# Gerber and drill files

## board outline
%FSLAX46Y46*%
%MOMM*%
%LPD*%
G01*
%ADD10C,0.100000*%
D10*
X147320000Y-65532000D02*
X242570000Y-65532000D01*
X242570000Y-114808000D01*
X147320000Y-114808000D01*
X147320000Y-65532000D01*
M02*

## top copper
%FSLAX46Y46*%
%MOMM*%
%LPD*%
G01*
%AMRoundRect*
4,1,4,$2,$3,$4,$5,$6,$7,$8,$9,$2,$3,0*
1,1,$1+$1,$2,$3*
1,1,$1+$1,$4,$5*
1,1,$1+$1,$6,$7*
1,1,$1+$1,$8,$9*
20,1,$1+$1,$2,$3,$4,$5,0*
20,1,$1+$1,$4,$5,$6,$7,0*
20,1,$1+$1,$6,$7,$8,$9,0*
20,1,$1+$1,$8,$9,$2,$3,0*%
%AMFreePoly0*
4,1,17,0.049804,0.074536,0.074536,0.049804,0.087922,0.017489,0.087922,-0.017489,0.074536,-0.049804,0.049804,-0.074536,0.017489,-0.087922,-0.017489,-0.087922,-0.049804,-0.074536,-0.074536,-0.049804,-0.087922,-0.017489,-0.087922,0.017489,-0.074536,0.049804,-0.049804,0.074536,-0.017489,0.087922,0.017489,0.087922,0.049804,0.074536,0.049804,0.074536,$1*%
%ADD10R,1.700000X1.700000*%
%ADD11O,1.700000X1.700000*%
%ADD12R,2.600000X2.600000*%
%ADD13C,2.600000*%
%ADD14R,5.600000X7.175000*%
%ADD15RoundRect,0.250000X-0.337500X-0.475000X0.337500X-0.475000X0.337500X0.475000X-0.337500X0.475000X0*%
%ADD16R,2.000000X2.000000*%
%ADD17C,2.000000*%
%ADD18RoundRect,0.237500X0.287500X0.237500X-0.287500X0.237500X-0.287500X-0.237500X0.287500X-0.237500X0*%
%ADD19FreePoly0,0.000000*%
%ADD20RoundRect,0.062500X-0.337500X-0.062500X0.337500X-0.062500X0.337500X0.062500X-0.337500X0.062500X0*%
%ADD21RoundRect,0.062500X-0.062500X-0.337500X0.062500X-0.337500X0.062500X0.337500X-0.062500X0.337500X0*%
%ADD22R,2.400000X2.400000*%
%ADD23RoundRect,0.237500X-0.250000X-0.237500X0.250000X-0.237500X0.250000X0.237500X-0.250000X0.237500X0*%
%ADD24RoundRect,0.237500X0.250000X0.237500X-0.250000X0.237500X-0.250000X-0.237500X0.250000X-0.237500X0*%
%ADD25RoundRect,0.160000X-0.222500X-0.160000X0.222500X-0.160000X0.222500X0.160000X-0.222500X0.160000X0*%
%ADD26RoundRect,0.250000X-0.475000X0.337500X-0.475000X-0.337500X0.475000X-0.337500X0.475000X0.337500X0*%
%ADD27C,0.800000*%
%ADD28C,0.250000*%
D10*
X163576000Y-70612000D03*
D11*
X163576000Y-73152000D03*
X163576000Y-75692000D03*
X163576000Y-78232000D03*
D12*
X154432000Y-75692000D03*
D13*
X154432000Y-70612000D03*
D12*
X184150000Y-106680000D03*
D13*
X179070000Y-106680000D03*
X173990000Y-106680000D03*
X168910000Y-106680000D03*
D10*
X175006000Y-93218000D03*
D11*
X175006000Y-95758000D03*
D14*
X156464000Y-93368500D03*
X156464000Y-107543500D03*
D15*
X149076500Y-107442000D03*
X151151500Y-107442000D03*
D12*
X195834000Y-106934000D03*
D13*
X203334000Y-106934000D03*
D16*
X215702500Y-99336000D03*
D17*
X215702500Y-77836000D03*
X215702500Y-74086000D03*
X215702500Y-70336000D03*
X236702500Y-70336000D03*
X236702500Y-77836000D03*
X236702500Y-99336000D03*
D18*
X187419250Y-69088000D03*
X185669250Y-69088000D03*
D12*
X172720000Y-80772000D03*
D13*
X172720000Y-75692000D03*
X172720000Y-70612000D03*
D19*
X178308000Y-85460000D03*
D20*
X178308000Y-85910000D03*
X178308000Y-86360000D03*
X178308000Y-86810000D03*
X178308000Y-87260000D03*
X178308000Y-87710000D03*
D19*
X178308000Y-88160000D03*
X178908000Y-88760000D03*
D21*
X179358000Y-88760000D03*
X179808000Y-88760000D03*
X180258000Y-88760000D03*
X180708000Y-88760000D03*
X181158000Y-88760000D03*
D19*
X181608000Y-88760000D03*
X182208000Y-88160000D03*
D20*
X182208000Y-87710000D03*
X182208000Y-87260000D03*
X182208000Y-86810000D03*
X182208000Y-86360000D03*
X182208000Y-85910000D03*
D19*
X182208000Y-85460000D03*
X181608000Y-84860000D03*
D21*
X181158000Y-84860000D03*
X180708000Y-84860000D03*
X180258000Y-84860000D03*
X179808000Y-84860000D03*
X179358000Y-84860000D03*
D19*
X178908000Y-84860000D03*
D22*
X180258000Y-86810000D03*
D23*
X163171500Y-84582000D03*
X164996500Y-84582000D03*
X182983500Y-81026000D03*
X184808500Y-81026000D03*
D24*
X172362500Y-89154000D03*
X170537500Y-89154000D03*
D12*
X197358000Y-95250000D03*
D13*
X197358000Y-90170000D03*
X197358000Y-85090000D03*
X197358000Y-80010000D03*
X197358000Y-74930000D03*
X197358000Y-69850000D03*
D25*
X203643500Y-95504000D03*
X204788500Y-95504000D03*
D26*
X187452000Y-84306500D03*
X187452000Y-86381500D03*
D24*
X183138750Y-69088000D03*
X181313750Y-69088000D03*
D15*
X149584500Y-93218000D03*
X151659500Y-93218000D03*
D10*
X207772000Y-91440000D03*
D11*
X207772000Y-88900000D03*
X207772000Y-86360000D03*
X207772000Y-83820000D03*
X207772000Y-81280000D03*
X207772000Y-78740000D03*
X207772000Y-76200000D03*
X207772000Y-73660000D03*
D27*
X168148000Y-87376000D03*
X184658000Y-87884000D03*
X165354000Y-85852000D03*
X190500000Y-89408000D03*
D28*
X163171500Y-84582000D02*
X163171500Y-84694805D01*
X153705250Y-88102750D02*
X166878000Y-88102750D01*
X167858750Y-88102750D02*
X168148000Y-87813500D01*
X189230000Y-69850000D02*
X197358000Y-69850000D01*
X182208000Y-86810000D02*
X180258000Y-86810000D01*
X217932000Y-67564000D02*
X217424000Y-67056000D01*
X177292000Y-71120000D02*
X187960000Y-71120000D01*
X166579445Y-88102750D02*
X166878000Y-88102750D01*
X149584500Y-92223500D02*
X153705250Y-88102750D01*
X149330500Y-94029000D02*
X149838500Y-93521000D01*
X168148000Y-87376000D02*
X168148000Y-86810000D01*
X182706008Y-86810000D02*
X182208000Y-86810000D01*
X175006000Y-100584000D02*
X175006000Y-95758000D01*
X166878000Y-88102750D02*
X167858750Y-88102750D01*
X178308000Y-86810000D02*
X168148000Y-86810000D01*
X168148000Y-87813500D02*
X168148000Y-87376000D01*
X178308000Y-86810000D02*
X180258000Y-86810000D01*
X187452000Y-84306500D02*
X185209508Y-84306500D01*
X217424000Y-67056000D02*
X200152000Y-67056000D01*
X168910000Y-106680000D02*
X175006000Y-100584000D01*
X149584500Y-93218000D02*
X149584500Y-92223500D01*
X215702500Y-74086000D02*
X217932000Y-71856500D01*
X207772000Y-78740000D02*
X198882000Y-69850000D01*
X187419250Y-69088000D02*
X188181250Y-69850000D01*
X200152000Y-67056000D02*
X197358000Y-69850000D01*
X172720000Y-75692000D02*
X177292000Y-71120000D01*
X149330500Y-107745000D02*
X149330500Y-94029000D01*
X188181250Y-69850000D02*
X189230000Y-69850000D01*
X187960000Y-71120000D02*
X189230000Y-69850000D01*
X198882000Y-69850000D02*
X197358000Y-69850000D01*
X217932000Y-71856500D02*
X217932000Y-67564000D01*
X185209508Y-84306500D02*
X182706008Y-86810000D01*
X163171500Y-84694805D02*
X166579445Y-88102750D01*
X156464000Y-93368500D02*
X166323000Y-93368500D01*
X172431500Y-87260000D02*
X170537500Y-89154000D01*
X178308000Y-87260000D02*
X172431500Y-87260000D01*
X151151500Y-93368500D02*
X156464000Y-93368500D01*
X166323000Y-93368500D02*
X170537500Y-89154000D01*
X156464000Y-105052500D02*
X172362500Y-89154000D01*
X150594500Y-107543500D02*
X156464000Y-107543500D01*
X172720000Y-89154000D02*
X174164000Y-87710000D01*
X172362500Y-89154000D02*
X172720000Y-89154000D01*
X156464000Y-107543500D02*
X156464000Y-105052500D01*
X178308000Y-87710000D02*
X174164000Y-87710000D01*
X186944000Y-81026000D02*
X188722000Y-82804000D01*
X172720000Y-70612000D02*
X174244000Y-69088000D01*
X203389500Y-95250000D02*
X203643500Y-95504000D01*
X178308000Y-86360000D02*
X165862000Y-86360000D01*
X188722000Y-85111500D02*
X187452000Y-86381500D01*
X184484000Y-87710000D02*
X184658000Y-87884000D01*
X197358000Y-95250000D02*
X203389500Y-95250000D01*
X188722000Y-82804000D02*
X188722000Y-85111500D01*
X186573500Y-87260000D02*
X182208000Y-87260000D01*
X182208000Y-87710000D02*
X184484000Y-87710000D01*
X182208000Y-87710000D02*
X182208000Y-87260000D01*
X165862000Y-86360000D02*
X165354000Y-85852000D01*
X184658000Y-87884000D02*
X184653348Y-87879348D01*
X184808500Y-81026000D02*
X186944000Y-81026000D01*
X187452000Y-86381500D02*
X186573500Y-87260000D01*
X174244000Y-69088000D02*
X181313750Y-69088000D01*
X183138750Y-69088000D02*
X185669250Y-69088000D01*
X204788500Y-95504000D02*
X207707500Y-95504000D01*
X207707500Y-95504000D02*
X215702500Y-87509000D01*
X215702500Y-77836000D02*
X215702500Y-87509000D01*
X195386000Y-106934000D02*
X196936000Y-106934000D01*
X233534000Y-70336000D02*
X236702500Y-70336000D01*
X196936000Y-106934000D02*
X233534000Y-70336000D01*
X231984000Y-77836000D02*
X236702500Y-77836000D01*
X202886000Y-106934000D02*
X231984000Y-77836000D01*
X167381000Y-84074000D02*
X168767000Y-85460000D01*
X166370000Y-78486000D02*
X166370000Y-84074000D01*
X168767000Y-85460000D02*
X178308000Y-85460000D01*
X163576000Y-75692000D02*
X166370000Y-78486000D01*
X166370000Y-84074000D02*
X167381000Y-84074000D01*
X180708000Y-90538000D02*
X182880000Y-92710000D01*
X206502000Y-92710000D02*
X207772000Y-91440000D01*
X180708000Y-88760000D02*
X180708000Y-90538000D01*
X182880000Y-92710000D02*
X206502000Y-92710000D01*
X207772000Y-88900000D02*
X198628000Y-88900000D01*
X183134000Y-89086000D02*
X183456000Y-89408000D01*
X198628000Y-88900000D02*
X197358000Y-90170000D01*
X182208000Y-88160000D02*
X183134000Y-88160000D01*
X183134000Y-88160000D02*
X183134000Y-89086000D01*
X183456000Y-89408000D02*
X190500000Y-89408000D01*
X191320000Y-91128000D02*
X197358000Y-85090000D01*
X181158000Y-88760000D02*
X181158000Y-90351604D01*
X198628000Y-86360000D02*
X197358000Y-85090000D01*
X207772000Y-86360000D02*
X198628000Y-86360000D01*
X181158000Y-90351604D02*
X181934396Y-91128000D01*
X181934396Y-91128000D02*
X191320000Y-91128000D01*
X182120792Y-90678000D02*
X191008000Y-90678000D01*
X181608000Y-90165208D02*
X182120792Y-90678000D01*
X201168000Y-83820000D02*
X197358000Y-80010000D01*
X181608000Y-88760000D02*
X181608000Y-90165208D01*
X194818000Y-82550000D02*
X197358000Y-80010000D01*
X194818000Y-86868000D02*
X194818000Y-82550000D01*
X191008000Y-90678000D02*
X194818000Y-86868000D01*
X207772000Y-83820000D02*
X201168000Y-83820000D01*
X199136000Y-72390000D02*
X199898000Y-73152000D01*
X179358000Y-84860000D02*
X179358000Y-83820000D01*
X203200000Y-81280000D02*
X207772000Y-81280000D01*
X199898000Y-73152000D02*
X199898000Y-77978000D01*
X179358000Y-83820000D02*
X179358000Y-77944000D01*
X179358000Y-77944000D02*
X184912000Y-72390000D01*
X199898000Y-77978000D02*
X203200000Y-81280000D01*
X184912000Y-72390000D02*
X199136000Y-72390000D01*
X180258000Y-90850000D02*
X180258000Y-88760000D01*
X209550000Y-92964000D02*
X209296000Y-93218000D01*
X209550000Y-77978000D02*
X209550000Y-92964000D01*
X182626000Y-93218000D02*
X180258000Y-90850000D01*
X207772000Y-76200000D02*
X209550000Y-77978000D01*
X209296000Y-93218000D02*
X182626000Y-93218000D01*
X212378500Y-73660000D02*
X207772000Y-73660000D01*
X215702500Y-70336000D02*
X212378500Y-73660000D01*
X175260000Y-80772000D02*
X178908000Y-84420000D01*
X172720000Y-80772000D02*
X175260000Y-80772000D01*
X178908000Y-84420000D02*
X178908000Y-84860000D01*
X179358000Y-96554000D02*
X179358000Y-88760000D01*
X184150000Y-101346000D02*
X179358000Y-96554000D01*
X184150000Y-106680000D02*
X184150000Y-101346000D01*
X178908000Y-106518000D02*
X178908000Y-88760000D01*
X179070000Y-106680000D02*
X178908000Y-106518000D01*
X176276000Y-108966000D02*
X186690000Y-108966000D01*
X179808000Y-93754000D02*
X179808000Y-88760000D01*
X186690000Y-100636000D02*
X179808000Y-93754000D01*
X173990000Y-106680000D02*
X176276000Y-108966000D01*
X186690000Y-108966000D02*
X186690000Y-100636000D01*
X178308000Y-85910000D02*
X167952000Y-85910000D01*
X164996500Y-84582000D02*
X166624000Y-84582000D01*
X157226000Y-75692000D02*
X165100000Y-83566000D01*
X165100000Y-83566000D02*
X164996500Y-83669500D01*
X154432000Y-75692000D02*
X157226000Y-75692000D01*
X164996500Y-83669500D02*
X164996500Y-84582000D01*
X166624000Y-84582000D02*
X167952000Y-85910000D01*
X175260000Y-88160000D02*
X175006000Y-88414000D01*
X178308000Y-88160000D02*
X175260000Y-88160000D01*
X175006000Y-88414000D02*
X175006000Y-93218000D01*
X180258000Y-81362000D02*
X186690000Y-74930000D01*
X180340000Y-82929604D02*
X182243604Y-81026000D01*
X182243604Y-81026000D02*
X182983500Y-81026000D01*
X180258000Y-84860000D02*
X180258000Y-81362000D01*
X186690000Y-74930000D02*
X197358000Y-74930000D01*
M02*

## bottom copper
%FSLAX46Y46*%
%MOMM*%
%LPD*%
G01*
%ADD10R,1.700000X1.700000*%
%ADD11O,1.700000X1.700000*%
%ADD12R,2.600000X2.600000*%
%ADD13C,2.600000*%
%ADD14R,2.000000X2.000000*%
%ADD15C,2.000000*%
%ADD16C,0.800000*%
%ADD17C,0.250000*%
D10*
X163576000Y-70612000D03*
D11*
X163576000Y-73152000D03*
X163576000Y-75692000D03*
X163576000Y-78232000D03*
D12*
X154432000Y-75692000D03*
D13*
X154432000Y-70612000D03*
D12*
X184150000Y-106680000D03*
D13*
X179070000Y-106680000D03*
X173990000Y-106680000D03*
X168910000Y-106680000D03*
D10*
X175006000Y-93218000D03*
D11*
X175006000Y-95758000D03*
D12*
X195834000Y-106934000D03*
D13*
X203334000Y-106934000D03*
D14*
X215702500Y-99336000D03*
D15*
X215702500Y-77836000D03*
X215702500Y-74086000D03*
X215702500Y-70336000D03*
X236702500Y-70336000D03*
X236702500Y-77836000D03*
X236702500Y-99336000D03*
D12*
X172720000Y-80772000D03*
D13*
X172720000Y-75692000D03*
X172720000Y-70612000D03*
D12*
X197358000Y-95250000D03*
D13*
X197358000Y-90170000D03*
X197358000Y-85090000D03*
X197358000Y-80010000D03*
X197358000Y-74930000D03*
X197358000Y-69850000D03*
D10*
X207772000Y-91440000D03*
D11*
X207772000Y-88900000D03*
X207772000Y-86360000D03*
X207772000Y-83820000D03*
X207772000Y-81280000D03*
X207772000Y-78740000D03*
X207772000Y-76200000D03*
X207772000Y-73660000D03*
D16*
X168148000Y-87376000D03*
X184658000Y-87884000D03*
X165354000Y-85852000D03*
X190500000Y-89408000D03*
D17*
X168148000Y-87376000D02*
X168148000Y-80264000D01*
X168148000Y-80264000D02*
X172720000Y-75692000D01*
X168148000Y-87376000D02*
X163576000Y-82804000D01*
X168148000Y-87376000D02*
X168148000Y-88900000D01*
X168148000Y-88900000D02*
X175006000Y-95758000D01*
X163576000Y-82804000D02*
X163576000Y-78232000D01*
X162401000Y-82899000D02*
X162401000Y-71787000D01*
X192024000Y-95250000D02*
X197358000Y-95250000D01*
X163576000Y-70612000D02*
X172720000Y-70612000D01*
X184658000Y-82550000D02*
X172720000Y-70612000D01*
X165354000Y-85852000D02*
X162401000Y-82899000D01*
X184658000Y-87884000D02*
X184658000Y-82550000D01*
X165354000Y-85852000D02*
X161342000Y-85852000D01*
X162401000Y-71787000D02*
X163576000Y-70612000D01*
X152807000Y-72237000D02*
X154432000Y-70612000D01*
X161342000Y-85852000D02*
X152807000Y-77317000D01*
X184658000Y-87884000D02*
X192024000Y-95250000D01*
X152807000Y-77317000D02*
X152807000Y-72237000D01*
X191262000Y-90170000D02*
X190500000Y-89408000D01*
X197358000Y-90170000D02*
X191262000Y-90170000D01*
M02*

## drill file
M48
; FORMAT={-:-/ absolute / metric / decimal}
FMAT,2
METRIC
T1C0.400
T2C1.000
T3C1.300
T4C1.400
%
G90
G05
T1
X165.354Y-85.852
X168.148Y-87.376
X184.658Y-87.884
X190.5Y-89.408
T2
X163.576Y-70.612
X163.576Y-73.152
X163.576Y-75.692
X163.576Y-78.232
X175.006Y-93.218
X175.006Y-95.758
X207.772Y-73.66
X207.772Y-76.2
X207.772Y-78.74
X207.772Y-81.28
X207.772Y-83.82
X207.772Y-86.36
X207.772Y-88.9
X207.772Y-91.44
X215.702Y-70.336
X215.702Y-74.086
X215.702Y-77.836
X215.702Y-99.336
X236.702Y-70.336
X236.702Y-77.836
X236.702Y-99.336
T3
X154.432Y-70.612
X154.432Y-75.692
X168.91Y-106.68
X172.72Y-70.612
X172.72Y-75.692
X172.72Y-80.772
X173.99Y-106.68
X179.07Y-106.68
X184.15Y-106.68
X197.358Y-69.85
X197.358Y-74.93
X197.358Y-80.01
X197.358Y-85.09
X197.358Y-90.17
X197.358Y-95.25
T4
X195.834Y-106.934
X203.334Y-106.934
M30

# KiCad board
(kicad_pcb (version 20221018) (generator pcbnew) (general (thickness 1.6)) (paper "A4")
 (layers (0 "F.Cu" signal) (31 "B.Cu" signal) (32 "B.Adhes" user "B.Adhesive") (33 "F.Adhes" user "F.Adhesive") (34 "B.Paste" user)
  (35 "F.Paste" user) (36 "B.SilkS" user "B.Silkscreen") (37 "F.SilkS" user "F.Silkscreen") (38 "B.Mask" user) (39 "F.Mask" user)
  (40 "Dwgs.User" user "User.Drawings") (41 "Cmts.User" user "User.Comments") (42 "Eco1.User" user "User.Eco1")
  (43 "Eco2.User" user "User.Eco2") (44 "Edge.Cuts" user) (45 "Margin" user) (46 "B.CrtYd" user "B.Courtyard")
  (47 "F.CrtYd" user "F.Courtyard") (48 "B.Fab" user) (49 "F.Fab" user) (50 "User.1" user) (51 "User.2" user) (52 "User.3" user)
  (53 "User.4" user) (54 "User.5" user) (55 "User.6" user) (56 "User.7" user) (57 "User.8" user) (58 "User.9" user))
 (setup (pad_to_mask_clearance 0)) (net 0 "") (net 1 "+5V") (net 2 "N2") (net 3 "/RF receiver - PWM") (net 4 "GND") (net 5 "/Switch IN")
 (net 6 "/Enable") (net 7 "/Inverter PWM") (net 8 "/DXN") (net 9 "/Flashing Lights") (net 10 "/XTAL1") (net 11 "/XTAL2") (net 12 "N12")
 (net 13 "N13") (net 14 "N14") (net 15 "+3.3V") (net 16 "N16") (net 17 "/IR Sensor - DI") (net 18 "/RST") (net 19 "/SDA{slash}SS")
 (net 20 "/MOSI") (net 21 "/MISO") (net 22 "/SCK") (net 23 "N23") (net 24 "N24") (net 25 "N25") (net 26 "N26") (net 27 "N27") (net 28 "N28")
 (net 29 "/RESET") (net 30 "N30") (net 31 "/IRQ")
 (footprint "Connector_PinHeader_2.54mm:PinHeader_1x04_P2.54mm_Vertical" (layer "F.Cu") (at 163.576 70.612)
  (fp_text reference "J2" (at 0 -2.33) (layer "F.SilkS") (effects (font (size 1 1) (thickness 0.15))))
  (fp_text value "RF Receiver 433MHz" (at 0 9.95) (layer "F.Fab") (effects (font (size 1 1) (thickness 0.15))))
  (pad "1" thru_hole rect (at 0 0) (size 1.7 1.7) (drill 1) (layers "*.Cu" "*.Mask") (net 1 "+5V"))
  (pad "2" thru_hole oval (at 0 2.54) (size 1.7 1.7) (drill 1) (layers "*.Cu" "*.Mask") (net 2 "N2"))
  (pad "3" thru_hole oval (at 0 5.08) (size 1.7 1.7) (drill 1) (layers "*.Cu" "*.Mask") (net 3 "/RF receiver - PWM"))
  (pad "4" thru_hole oval (at 0 7.62) (size 1.7 1.7) (drill 1) (layers "*.Cu" "*.Mask") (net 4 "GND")))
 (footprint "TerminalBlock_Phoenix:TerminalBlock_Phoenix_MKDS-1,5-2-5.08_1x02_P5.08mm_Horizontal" (layer "F.Cu") (at 154.432 75.692 90)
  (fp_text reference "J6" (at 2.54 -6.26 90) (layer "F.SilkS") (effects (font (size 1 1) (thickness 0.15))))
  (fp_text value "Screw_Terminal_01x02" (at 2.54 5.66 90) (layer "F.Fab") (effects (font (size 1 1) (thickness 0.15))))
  (pad "1" thru_hole rect (at 0 0 90) (size 2.6 2.6) (drill 1.3) (layers "*.Cu" "*.Mask") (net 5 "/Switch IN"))
  (pad "2" thru_hole circle (at 5.08 0 90) (size 2.6 2.6) (drill 1.3) (layers "*.Cu" "*.Mask") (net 1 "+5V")))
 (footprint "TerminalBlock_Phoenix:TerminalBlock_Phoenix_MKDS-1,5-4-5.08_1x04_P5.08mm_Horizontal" (layer "F.Cu") (at 184.15 106.68 180)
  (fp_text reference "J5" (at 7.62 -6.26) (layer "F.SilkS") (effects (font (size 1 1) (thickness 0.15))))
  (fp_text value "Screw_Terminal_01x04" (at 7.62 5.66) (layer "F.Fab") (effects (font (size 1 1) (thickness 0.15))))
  (pad "1" thru_hole rect (at 0 0 180) (size 2.6 2.6) (drill 1.3) (layers "*.Cu" "*.Mask") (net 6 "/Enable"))
  (pad "2" thru_hole circle (at 5.08 0 180) (size 2.6 2.6) (drill 1.3) (layers "*.Cu" "*.Mask") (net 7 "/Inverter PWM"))
  (pad "3" thru_hole circle (at 10.16 0 180) (size 2.6 2.6) (drill 1.3) (layers "*.Cu" "*.Mask") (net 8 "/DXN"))
  (pad "4" thru_hole circle (at 15.24 0 180) (size 2.6 2.6) (drill 1.3) (layers "*.Cu" "*.Mask") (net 4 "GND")))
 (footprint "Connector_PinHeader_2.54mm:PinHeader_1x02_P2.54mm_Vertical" (layer "F.Cu") (at 175.006 93.218)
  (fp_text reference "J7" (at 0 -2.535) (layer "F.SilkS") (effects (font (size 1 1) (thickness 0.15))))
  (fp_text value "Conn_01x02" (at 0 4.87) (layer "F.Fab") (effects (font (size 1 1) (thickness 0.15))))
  (pad "1" thru_hole rect (at 0 0) (size 1.7 1.7) (drill 1) (layers "*.Cu" "*.Mask") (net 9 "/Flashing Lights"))
  (pad "2" thru_hole oval (at 0 2.54) (size 1.7 1.7) (drill 1) (layers "*.Cu" "*.Mask") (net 4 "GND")))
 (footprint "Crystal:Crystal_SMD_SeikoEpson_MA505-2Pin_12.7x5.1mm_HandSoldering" (layer "F.Cu") (at 156.464 100.456 -90)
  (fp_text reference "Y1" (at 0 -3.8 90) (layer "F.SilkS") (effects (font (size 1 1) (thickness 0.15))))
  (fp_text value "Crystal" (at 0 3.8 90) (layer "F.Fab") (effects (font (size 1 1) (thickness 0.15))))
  (pad "1" smd rect (at -7.0875 0 270) (size 7.175 5.6) (layers "F.Cu" "F.Paste" "F.Mask") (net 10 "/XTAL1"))
  (pad "2" smd rect (at 7.0875 0 270) (size 7.175 5.6) (layers "F.Cu" "F.Paste" "F.Mask") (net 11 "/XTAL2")))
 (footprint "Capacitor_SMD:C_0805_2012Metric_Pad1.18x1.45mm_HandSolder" (layer "F.Cu") (at 150.114 107.442)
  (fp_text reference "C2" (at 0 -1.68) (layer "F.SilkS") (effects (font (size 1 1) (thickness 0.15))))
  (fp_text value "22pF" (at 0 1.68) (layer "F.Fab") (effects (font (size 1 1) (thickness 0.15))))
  (pad "1" smd roundrect (at -1.0375 0) (size 1.175 1.45) (layers "F.Cu" "F.Paste" "F.Mask") (roundrect_rratio 0.212766) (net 4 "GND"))
  (pad "2" smd roundrect (at 1.0375 0) (size 1.175 1.45) (layers "F.Cu" "F.Paste" "F.Mask") (roundrect_rratio 0.212766) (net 11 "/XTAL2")))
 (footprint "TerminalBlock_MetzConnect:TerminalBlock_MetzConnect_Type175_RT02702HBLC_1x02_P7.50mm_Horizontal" (layer "F.Cu")
  (at 195.834 106.934)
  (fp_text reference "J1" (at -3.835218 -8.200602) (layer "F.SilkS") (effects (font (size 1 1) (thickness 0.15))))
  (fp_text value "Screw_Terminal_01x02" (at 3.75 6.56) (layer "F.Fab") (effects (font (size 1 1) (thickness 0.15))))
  (pad "1" thru_hole rect (at 0 0) (size 2.6 2.6) (drill 1.4) (layers "*.Cu" "*.Mask") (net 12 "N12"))
  (pad "2" thru_hole circle (at 7.5 0) (size 2.6 2.6) (drill 1.4) (layers "*.Cu" "*.Mask") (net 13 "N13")))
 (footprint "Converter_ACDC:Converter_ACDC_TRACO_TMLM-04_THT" (layer "F.Cu") (at 215.7025 99.336 90)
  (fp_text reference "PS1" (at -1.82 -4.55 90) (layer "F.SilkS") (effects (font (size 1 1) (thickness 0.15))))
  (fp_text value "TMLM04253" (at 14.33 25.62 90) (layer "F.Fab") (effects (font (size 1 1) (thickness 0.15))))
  (pad "1" thru_hole rect (at 0 0 90) (size 2 2) (drill 1) (layers "*.Cu" "*.Mask"))
  (pad "2" thru_hole circle (at 21.5 0 90) (size 2 2) (drill 1) (layers "*.Cu" "*.Mask") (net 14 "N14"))
  (pad "3" thru_hole circle (at 25.25 0 90) (size 2 2) (drill 1) (layers "*.Cu" "*.Mask") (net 4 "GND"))
  (pad "4" thru_hole circle (at 29 0 90) (size 2 2) (drill 1) (layers "*.Cu" "*.Mask") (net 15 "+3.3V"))
  (pad "5" thru_hole circle (at 29 21 90) (size 2 2) (drill 1) (layers "*.Cu" "*.Mask") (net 12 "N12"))
  (pad "6" thru_hole circle (at 21.5 21 90) (size 2 2) (drill 1) (layers "*.Cu" "*.Mask") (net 13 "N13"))
  (pad "7" thru_hole circle (at 0 21 90) (size 2 2) (drill 1) (layers "*.Cu" "*.Mask")))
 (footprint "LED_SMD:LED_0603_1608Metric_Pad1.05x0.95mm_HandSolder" (layer "F.Cu") (at 186.54425 69.088 180)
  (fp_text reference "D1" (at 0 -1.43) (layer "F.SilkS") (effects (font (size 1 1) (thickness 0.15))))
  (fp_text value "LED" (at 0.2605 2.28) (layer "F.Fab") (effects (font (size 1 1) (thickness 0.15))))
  (pad "1" smd roundrect (at -0.875 0 180) (size 1.05 0.95) (layers "F.Cu" "F.Paste" "F.Mask") (roundrect_rratio 0.25) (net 4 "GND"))
  (pad "2" smd roundrect (at 0.875 0 180) (size 1.05 0.95) (layers "F.Cu" "F.Paste" "F.Mask") (roundrect_rratio 0.25) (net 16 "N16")))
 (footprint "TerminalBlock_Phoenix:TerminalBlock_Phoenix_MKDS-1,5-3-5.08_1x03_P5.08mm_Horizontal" (layer "F.Cu") (at 172.72 80.772 90)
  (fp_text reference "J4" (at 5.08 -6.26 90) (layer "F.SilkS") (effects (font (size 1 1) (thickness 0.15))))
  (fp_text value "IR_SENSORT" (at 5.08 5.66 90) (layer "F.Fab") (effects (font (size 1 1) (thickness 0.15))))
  (pad "1" thru_hole rect (at 0 0 90) (size 2.6 2.6) (drill 1.3) (layers "*.Cu" "*.Mask") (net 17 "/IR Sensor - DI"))
  (pad "2" thru_hole circle (at 5.08 0 90) (size 2.6 2.6) (drill 1.3) (layers "*.Cu" "*.Mask") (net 4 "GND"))
  (pad "3" thru_hole circle (at 10.16 0 90) (size 2.6 2.6) (drill 1.3) (layers "*.Cu" "*.Mask") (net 1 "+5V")))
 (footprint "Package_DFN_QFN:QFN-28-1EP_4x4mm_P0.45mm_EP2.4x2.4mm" (layer "F.Cu") (at 180.258 86.81)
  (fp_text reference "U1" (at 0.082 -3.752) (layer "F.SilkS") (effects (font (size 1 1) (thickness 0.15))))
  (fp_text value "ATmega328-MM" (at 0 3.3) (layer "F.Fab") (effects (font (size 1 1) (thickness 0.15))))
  (pad "" smd roundrect (at -0.6 -0.6) (size 0.97 0.97) (layers "F.Paste") (roundrect_rratio 0.25))
  (pad "" smd roundrect (at -0.6 0.6) (size 0.97 0.97) (layers "F.Paste") (roundrect_rratio 0.25))
  (pad "" smd roundrect (at 0.6 -0.6) (size 0.97 0.97) (layers "F.Paste") (roundrect_rratio 0.25))
  (pad "" smd roundrect (at 0.6 0.6) (size 0.97 0.97) (layers "F.Paste") (roundrect_rratio 0.25))
  (pad "1" smd custom (at -1.95 -1.35) (size 0.179289 0.179289) (layers "F.Cu" "F.Paste" "F.Mask") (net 3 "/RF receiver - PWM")
   (thermal_bridge_angle 45) (options (clearance outline) (anchor circle)) (primitives))
  (pad "2" smd roundrect (at -1.95 -0.9) (size 0.8 0.25) (layers "F.Cu" "F.Paste" "F.Mask") (roundrect_rratio 0.25) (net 5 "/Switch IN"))
  (pad "3" smd roundrect (at -1.95 -0.45) (size 0.8 0.25) (layers "F.Cu" "F.Paste" "F.Mask") (roundrect_rratio 0.25) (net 1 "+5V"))
  (pad "4" smd roundrect (at -1.95 0) (size 0.8 0.25) (layers "F.Cu" "F.Paste" "F.Mask") (roundrect_rratio 0.25) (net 4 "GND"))
  (pad "5" smd roundrect (at -1.95 0.45) (size 0.8 0.25) (layers "F.Cu" "F.Paste" "F.Mask") (roundrect_rratio 0.25) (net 10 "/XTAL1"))
  (pad "6" smd roundrect (at -1.95 0.9) (size 0.8 0.25) (layers "F.Cu" "F.Paste" "F.Mask") (roundrect_rratio 0.25) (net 11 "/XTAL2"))
  (pad "7" smd custom (at -1.95 1.35) (size 0.179289 0.179289) (layers "F.Cu" "F.Paste" "F.Mask") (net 9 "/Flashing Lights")
   (thermal_bridge_angle 45) (options (clearance outline) (anchor circle)) (primitives))
  (pad "8" smd custom (at -1.35 1.95) (size 0.179289 0.179289) (layers "F.Cu" "F.Paste" "F.Mask") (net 7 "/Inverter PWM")
   (thermal_bridge_angle 45) (options (clearance outline) (anchor circle)) (primitives))
  (pad "9" smd roundrect (at -0.9 1.95) (size 0.25 0.8) (layers "F.Cu" "F.Paste" "F.Mask") (roundrect_rratio 0.25) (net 6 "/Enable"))
  (pad "10" smd roundrect (at -0.45 1.95) (size 0.25 0.8) (layers "F.Cu" "F.Paste" "F.Mask") (roundrect_rratio 0.25) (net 8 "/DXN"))
  (pad "11" smd roundrect (at 0 1.95) (size 0.25 0.8) (layers "F.Cu" "F.Paste" "F.Mask") (roundrect_rratio 0.25) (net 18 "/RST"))
  (pad "12" smd roundrect (at 0.45 1.95) (size 0.25 0.8) (layers "F.Cu" "F.Paste" "F.Mask") (roundrect_rratio 0.25) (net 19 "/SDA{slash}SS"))
  (pad "13" smd roundrect (at 0.9 1.95) (size 0.25 0.8) (layers "F.Cu" "F.Paste" "F.Mask") (roundrect_rratio 0.25) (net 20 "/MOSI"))
  (pad "14" smd custom (at 1.35 1.95) (size 0.179289 0.179289) (layers "F.Cu" "F.Paste" "F.Mask") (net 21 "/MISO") (thermal_bridge_angle 45)
   (options (clearance outline) (anchor circle)) (primitives))
  (pad "15" smd custom (at 1.95 1.35) (size 0.179289 0.179289) (layers "F.Cu" "F.Paste" "F.Mask") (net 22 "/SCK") (thermal_bridge_angle 45)
   (options (clearance outline) (anchor circle)) (primitives))
  (pad "16" smd roundrect (at 1.95 0.9) (size 0.8 0.25) (layers "F.Cu" "F.Paste" "F.Mask") (roundrect_rratio 0.25) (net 1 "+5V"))
  (pad "17" smd roundrect (at 1.95 0.45) (size 0.8 0.25) (layers "F.Cu" "F.Paste" "F.Mask") (roundrect_rratio 0.25) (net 1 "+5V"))
  (pad "18" smd roundrect (at 1.95 0) (size 0.8 0.25) (layers "F.Cu" "F.Paste" "F.Mask") (roundrect_rratio 0.25) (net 4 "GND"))
  (pad "19" smd roundrect (at 1.95 -0.45) (size 0.8 0.25) (layers "F.Cu" "F.Paste" "F.Mask") (roundrect_rratio 0.25) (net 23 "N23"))
  (pad "20" smd roundrect (at 1.95 -0.9) (size 0.8 0.25) (layers "F.Cu" "F.Paste" "F.Mask") (roundrect_rratio 0.25) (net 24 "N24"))
  (pad "21" smd custom (at 1.95 -1.35) (size 0.179289 0.179289) (layers "F.Cu" "F.Paste" "F.Mask") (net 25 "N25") (thermal_bridge_angle 45)
   (options (clearance outline) (anchor circle)) (primitives))
  (pad "22" smd custom (at 1.35 -1.95) (size 0.179289 0.179289) (layers "F.Cu" "F.Paste" "F.Mask") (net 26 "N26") (thermal_bridge_angle 45)
   (options (clearance outline) (anchor circle)) (primitives))
  (pad "23" smd roundrect (at 0.9 -1.95) (size 0.25 0.8) (layers "F.Cu" "F.Paste" "F.Mask") (roundrect_rratio 0.25) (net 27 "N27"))
  (pad "24" smd roundrect (at 0.45 -1.95) (size 0.25 0.8) (layers "F.Cu" "F.Paste" "F.Mask") (roundrect_rratio 0.25) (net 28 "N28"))
  (pad "25" smd roundrect (at 0 -1.95) (size 0.25 0.8) (layers "F.Cu" "F.Paste" "F.Mask") (roundrect_rratio 0.25) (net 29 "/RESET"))
  (pad "26" smd roundrect (at -0.45 -1.95) (size 0.25 0.8) (layers "F.Cu" "F.Paste" "F.Mask") (roundrect_rratio 0.25) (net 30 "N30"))
  (pad "27" smd roundrect (at -0.9 -1.95) (size 0.25 0.8) (layers "F.Cu" "F.Paste" "F.Mask") (roundrect_rratio 0.25) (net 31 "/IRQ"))
  (pad "28" smd custom (at -1.35 -1.95) (size 0.179289 0.179289) (layers "F.Cu" "F.Paste" "F.Mask") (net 17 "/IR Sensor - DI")
   (thermal_bridge_angle 45) (options (clearance outline) (anchor circle)) (primitives))
  (pad "29" smd rect (at 0 0) (size 2.4 2.4) (layers "F.Cu" "F.Mask") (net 4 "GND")))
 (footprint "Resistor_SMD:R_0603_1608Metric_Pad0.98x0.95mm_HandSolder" (layer "F.Cu") (at 164.084 84.582)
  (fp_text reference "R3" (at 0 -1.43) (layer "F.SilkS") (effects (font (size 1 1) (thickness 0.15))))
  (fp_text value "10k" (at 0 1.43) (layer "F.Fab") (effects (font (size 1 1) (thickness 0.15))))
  (pad "1" smd roundrect (at -0.9125 0) (size 0.975 0.95) (layers "F.Cu" "F.Paste" "F.Mask") (roundrect_rratio 0.25) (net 4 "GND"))
  (pad "2" smd roundrect (at 0.9125 0) (size 0.975 0.95) (layers "F.Cu" "F.Paste" "F.Mask") (roundrect_rratio 0.25) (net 5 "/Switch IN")))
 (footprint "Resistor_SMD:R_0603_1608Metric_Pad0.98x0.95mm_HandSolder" (layer "F.Cu") (at 183.896 81.026)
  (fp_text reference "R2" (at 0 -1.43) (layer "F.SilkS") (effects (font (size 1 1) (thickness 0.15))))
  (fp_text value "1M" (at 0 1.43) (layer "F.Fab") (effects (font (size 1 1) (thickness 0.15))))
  (pad "1" smd roundrect (at -0.9125 0) (size 0.975 0.95) (layers "F.Cu" "F.Paste" "F.Mask") (roundrect_rratio 0.25) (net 29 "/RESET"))
  (pad "2" smd roundrect (at 0.9125 0) (size 0.975 0.95) (layers "F.Cu" "F.Paste" "F.Mask") (roundrect_rratio 0.25) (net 1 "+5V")))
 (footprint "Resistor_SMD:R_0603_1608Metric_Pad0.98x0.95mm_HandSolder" (layer "F.Cu") (at 171.45 89.154 180)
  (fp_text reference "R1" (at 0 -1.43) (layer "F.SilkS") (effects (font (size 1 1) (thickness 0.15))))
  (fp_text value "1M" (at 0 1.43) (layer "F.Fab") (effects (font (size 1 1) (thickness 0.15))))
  (pad "1" smd roundrect (at -0.9125 0 180) (size 0.975 0.95) (layers "F.Cu" "F.Paste" "F.Mask") (roundrect_rratio 0.25) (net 11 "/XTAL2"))
  (pad "2" smd roundrect (at 0.9125 0 180) (size 0.975 0.95) (layers "F.Cu" "F.Paste" "F.Mask") (roundrect_rratio 0.25) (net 10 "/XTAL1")))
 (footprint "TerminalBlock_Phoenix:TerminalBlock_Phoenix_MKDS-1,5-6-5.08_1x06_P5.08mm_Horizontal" (layer "F.Cu") (at 197.358 95.25 90)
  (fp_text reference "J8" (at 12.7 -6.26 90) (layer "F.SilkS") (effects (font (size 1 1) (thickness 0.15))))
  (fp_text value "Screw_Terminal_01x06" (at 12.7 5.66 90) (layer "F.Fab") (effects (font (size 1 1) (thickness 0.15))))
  (pad "1" thru_hole rect (at 0 0 90) (size 2.6 2.6) (drill 1.3) (layers "*.Cu" "*.Mask") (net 1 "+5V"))
  (pad "2" thru_hole circle (at 5.08 0 90) (size 2.6 2.6) (drill 1.3) (layers "*.Cu" "*.Mask") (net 22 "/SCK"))
  (pad "3" thru_hole circle (at 10.16 0 90) (size 2.6 2.6) (drill 1.3) (layers "*.Cu" "*.Mask") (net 20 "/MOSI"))
  (pad "4" thru_hole circle (at 15.24 0 90) (size 2.6 2.6) (drill 1.3) (layers "*.Cu" "*.Mask") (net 21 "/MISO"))
  (pad "5" thru_hole circle (at 20.32 0 90) (size 2.6 2.6) (drill 1.3) (layers "*.Cu" "*.Mask") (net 29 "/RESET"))
  (pad "6" thru_hole circle (at 25.4 0 90) (size 2.6 2.6) (drill 1.3) (layers "*.Cu" "*.Mask") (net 4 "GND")))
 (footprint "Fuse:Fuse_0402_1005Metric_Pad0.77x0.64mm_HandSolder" (layer "F.Cu") (at 204.216 95.504)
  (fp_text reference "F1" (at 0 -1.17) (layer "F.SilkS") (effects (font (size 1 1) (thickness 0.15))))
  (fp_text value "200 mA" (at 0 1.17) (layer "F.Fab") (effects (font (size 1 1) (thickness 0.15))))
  (pad "1" smd roundrect (at -0.5725 0) (size 0.765 0.64) (layers "F.Cu" "F.Paste" "F.Mask") (roundrect_rratio 0.25) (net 1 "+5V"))
  (pad "2" smd roundrect (at 0.5725 0) (size 0.765 0.64) (layers "F.Cu" "F.Paste" "F.Mask") (roundrect_rratio 0.25) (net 14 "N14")))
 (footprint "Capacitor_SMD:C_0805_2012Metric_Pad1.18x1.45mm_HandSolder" (layer "F.Cu") (at 187.452 85.344 -90)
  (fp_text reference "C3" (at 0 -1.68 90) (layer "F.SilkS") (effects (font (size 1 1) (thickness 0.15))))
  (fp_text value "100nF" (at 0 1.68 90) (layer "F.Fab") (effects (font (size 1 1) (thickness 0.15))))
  (pad "1" smd roundrect (at -1.0375 0 270) (size 1.175 1.45) (layers "F.Cu" "F.Paste" "F.Mask") (roundrect_rratio 0.212766) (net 4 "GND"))
  (pad "2" smd roundrect (at 1.0375 0 270) (size 1.175 1.45) (layers "F.Cu" "F.Paste" "F.Mask") (roundrect_rratio 0.212766) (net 1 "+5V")))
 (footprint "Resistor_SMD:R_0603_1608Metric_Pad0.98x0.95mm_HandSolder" (layer "F.Cu") (at 182.22625 69.088 180)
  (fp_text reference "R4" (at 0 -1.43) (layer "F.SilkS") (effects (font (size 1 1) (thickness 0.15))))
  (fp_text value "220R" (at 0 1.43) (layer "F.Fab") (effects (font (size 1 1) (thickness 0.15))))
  (pad "1" smd roundrect (at -0.9125 0 180) (size 0.975 0.95) (layers "F.Cu" "F.Paste" "F.Mask") (roundrect_rratio 0.25) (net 16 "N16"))
  (pad "2" smd roundrect (at 0.9125 0 180) (size 0.975 0.95) (layers "F.Cu" "F.Paste" "F.Mask") (roundrect_rratio 0.25) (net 1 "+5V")))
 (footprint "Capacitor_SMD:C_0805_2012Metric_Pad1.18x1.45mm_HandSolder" (layer "F.Cu") (at 150.622 93.218)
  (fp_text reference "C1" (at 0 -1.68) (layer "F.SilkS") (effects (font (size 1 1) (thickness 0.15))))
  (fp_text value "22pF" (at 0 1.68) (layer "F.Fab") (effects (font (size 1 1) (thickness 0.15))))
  (pad "1" smd roundrect (at -1.0375 0) (size 1.175 1.45) (layers "F.Cu" "F.Paste" "F.Mask") (roundrect_rratio 0.212766) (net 4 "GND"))
  (pad "2" smd roundrect (at 1.0375 0) (size 1.175 1.45) (layers "F.Cu" "F.Paste" "F.Mask") (roundrect_rratio 0.212766) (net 10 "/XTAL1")))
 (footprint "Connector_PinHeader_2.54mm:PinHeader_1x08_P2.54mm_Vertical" (layer "F.Cu") (at 207.772 91.44 180)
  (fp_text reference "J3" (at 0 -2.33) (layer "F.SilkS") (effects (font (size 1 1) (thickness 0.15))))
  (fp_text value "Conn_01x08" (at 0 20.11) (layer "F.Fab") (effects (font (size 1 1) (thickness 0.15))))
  (pad "1" thru_hole rect (at 0 0 180) (size 1.7 1.7) (drill 1) (layers "*.Cu" "*.Mask") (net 19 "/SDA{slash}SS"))
  (pad "2" thru_hole oval (at 0 2.54 180) (size 1.7 1.7) (drill 1) (layers "*.Cu" "*.Mask") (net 22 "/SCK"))
  (pad "3" thru_hole oval (at 0 5.08 180) (size 1.7 1.7) (drill 1) (layers "*.Cu" "*.Mask") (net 20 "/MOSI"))
  (pad "4" thru_hole oval (at 0 7.62 180) (size 1.7 1.7) (drill 1) (layers "*.Cu" "*.Mask") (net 21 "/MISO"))
  (pad "5" thru_hole oval (at 0 10.16 180) (size 1.7 1.7) (drill 1) (layers "*.Cu" "*.Mask") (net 31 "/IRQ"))
  (pad "6" thru_hole oval (at 0 12.7 180) (size 1.7 1.7) (drill 1) (layers "*.Cu" "*.Mask") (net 4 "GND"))
  (pad "7" thru_hole oval (at 0 15.24 180) (size 1.7 1.7) (drill 1) (layers "*.Cu" "*.Mask") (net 18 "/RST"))
  (pad "8" thru_hole oval (at 0 17.78 180) (size 1.7 1.7) (drill 1) (layers "*.Cu" "*.Mask") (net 15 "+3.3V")))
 (gr_rect (start 147.32 65.532) (end 242.57 114.808) (stroke (width 0.1) (type default)) (fill none) (layer "Edge.Cuts"))
 (segment (start 163.1715 84.582) (end 163.1715 84.694805) (width 0.25) (layer "F.Cu") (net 4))
 (segment (start 153.70525 88.10275) (end 166.878 88.10275) (width 0.25) (layer "F.Cu") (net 4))
 (segment (start 167.85875 88.10275) (end 168.148 87.8135) (width 0.25) (layer "F.Cu") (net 4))
 (segment (start 189.23 69.85) (end 197.358 69.85) (width 0.25) (layer "F.Cu") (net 4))
 (segment (start 182.208 86.81) (end 180.258 86.81) (width 0.25) (layer "F.Cu") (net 4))
 (segment (start 217.932 67.564) (end 217.424 67.056) (width 0.25) (layer "F.Cu") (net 4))
 (segment (start 177.292 71.12) (end 187.96 71.12) (width 0.25) (layer "F.Cu") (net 4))
 (segment (start 166.579445 88.10275) (end 166.878 88.10275) (width 0.25) (layer "F.Cu") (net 4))
 (segment (start 149.5845 92.2235) (end 153.70525 88.10275) (width 0.25) (layer "F.Cu") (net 4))
 (segment (start 149.3305 94.029) (end 149.8385 93.521) (width 0.25) (layer "F.Cu") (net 4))
 (segment (start 168.148 87.376) (end 168.148 86.81) (width 0.25) (layer "F.Cu") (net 4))
 (segment (start 182.706008 86.81) (end 182.208 86.81) (width 0.25) (layer "F.Cu") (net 4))
 (segment (start 175.006 100.584) (end 175.006 95.758) (width 0.25) (layer "F.Cu") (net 4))
 (segment (start 166.878 88.10275) (end 167.85875 88.10275) (width 0.25) (layer "F.Cu") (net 4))
 (segment (start 178.308 86.81) (end 168.148 86.81) (width 0.25) (layer "F.Cu") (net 4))
 (segment (start 168.148 87.8135) (end 168.148 87.376) (width 0.25) (layer "F.Cu") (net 4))
 (segment (start 178.308 86.81) (end 180.258 86.81) (width 0.25) (layer "F.Cu") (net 4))
 (segment (start 187.452 84.3065) (end 185.209508 84.3065) (width 0.25) (layer "F.Cu") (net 4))
 (segment (start 217.424 67.056) (end 200.152 67.056) (width 0.25) (layer "F.Cu") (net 4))
 (segment (start 168.91 106.68) (end 175.006 100.584) (width 0.25) (layer "F.Cu") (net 4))
 (segment (start 149.5845 93.218) (end 149.5845 92.2235) (width 0.25) (layer "F.Cu") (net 4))
 (segment (start 215.7025 74.086) (end 217.932 71.8565) (width 0.25) (layer "F.Cu") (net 4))
 (segment (start 207.772 78.74) (end 198.882 69.85) (width 0.25) (layer "F.Cu") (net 4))
 (segment (start 187.41925 69.088) (end 188.18125 69.85) (width 0.25) (layer "F.Cu") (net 4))
 (segment (start 200.152 67.056) (end 197.358 69.85) (width 0.25) (layer "F.Cu") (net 4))
 (segment (start 172.72 75.692) (end 177.292 71.12) (width 0.25) (layer "F.Cu") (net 4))
 (segment (start 149.3305 107.745) (end 149.3305 94.029) (width 0.25) (layer "F.Cu") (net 4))
 (segment (start 188.18125 69.85) (end 189.23 69.85) (width 0.25) (layer "F.Cu") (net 4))
 (segment (start 187.96 71.12) (end 189.23 69.85) (width 0.25) (layer "F.Cu") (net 4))
 (segment (start 198.882 69.85) (end 197.358 69.85) (width 0.25) (layer "F.Cu") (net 4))
 (segment (start 217.932 71.8565) (end 217.932 67.564) (width 0.25) (layer "F.Cu") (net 4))
 (segment (start 185.209508 84.3065) (end 182.706008 86.81) (width 0.25) (layer "F.Cu") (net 4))
 (segment (start 163.1715 84.694805) (end 166.579445 88.10275) (width 0.25) (layer "F.Cu") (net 4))
 (via (at 168.148 87.376) (size 0.8) (drill 0.4) (layers "F.Cu" "B.Cu") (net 4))
 (segment (start 168.148 87.376) (end 168.148 80.264) (width 0.25) (layer "B.Cu") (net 4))
 (segment (start 168.148 80.264) (end 172.72 75.692) (width 0.25) (layer "B.Cu") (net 4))
 (segment (start 168.148 87.376) (end 163.576 82.804) (width 0.25) (layer "B.Cu") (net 4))
 (segment (start 168.148 87.376) (end 168.148 88.9) (width 0.25) (layer "B.Cu") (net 4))
 (segment (start 168.148 88.9) (end 175.006 95.758) (width 0.25) (layer "B.Cu") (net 4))
 (segment (start 163.576 82.804) (end 163.576 78.232) (width 0.25) (layer "B.Cu") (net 4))
 (segment (start 156.464 93.3685) (end 166.323 93.3685) (width 0.25) (layer "F.Cu") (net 10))
 (segment (start 172.4315 87.26) (end 170.5375 89.154) (width 0.25) (layer "F.Cu") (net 10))
 (segment (start 178.308 87.26) (end 172.4315 87.26) (width 0.25) (layer "F.Cu") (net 10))
 (segment (start 151.1515 93.3685) (end 156.464 93.3685) (width 0.25) (layer "F.Cu") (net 10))
 (segment (start 166.323 93.3685) (end 170.5375 89.154) (width 0.25) (layer "F.Cu") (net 10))
 (segment (start 156.464 105.0525) (end 172.3625 89.154) (width 0.25) (layer "F.Cu") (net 11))
 (segment (start 150.5945 107.5435) (end 156.464 107.5435) (width 0.25) (layer "F.Cu") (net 11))
 (segment (start 172.72 89.154) (end 174.164 87.71) (width 0.25) (layer "F.Cu") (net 11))
 (segment (start 172.3625 89.154) (end 172.72 89.154) (width 0.25) (layer "F.Cu") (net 11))
 (segment (start 156.464 107.5435) (end 156.464 105.0525) (width 0.25) (layer "F.Cu") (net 11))
 (segment (start 178.308 87.71) (end 174.164 87.71) (width 0.25) (layer "F.Cu") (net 11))
 (segment (start 186.944 81.026) (end 188.722 82.804) (width 0.25) (layer "F.Cu") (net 1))
 (segment (start 172.72 70.612) (end 174.244 69.088) (width 0.25) (layer "F.Cu") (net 1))
 (segment (start 203.3895 95.25) (end 203.6435 95.504) (width 0.25) (layer "F.Cu") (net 1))
 (segment (start 178.308 86.36) (end 165.862 86.36) (width 0.25) (layer "F.Cu") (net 1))
 (segment (start 188.722 85.1115) (end 187.452 86.3815) (width 0.25) (layer "F.Cu") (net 1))
 (segment (start 184.484 87.71) (end 184.658 87.884) (width 0.25) (layer "F.Cu") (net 1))
 (segment (start 197.358 95.25) (end 203.3895 95.25) (width 0.25) (layer "F.Cu") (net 1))
 (segment (start 188.722 82.804) (end 188.722 85.1115) (width 0.25) (layer "F.Cu") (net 1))
 (segment (start 186.5735 87.26) (end 182.208 87.26) (width 0.25) (layer "F.Cu") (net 1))
 (segment (start 182.208 87.71) (end 184.484 87.71) (width 0.25) (layer "F.Cu") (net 1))
 (segment (start 182.208 87.71) (end 182.208 87.26) (width 0.25) (layer "F.Cu") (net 1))
 (segment (start 165.862 86.36) (end 165.354 85.852) (width 0.25) (layer "F.Cu") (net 1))
 (segment (start 184.658 87.884) (end 184.653348 87.879348) (width 0.25) (layer "F.Cu") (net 1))
 (segment (start 184.8085 81.026) (end 186.944 81.026) (width 0.25) (layer "F.Cu") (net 1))
 (segment (start 187.452 86.3815) (end 186.5735 87.26) (width 0.25) (layer "F.Cu") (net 1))
 (segment (start 174.244 69.088) (end 181.31375 69.088) (width 0.25) (layer "F.Cu") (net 1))
 (via (at 184.658 87.884) (size 0.8) (drill 0.4) (layers "F.Cu" "B.Cu") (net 1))
 (via (at 165.354 85.852) (size 0.8) (drill 0.4) (layers "F.Cu" "B.Cu") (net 1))
 (segment (start 162.401 82.899) (end 162.401 71.787) (width 0.25) (layer "B.Cu") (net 1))
 (segment (start 192.024 95.25) (end 197.358 95.25) (width 0.25) (layer "B.Cu") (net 1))
 (segment (start 163.576 70.612) (end 172.72 70.612) (width 0.25) (layer "B.Cu") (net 1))
 (segment (start 184.658 82.55) (end 172.72 70.612) (width 0.25) (layer "B.Cu") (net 1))
 (segment (start 165.354 85.852) (end 162.401 82.899) (width 0.25) (layer "B.Cu") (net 1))
 (segment (start 184.658 87.884) (end 184.658 82.55) (width 0.25) (layer "B.Cu") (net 1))
 (segment (start 165.354 85.852) (end 161.342 85.852) (width 0.25) (layer "B.Cu") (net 1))
 (segment (start 162.401 71.787) (end 163.576 70.612) (width 0.25) (layer "B.Cu") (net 1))
 (segment (start 152.807 72.237) (end 154.432 70.612) (width 0.25) (layer "B.Cu") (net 1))
 (segment (start 161.342 85.852) (end 152.807 77.317) (width 0.25) (layer "B.Cu") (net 1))
 (segment (start 184.658 87.884) (end 192.024 95.25) (width 0.25) (layer "B.Cu") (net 1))
 (segment (start 152.807 77.317) (end 152.807 72.237) (width 0.25) (layer "B.Cu") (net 1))
 (segment (start 183.13875 69.088) (end 185.66925 69.088) (width 0.25) (layer "F.Cu") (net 16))
 (segment (start 204.7885 95.504) (end 207.7075 95.504) (width 0.25) (layer "F.Cu") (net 14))
 (segment (start 207.7075 95.504) (end 215.7025 87.509) (width 0.25) (layer "F.Cu") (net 14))
 (segment (start 215.7025 77.836) (end 215.7025 87.509) (width 0.25) (layer "F.Cu") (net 14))
 (segment (start 195.386 106.934) (end 196.936 106.934) (width 0.25) (layer "F.Cu") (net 12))
 (segment (start 233.534 70.336) (end 236.7025 70.336) (width 0.25) (layer "F.Cu") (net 12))
 (segment (start 196.936 106.934) (end 233.534 70.336) (width 0.25) (layer "F.Cu") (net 12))
 (segment (start 231.984 77.836) (end 236.7025 77.836) (width 0.25) (layer "F.Cu") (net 13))
 (segment (start 202.886 106.934) (end 231.984 77.836) (width 0.25) (layer "F.Cu") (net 13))
 (segment (start 167.381 84.074) (end 168.767 85.46) (width 0.25) (layer "F.Cu") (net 3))
 (segment (start 166.37 78.486) (end 166.37 84.074) (width 0.25) (layer "F.Cu") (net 3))
 (segment (start 168.767 85.46) (end 178.308 85.46) (width 0.25) (layer "F.Cu") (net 3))
 (segment (start 163.576 75.692) (end 166.37 78.486) (width 0.25) (layer "F.Cu") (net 3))
 (segment (start 166.37 84.074) (end 167.381 84.074) (width 0.25) (layer "F.Cu") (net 3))
 (segment (start 180.708 90.538) (end 182.88 92.71) (width 0.25) (layer "F.Cu") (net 19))
 (segment (start 206.502 92.71) (end 207.772 91.44) (width 0.25) (layer "F.Cu") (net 19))
 (segment (start 180.708 88.76) (end 180.708 90.538) (width 0.25) (layer "F.Cu") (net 19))
 (segment (start 182.88 92.71) (end 206.502 92.71) (width 0.25) (layer "F.Cu") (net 19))
 (segment (start 207.772 88.9) (end 198.628 88.9) (width 0.25) (layer "F.Cu") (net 22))
 (segment (start 183.134 89.086) (end 183.456 89.408) (width 0.25) (layer "F.Cu") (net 22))
 (segment (start 198.628 88.9) (end 197.358 90.17) (width 0.25) (layer "F.Cu") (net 22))
 (segment (start 182.208 88.16) (end 183.134 88.16) (width 0.25) (layer "F.Cu") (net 22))
 (segment (start 183.134 88.16) (end 183.134 89.086) (width 0.25) (layer "F.Cu") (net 22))
 (segment (start 183.456 89.408) (end 190.5 89.408) (width 0.25) (layer "F.Cu") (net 22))
 (via (at 190.5 89.408) (size 0.8) (drill 0.4) (layers "F.Cu" "B.Cu") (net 22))
 (segment (start 191.262 90.17) (end 190.5 89.408) (width 0.25) (layer "B.Cu") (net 22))
 (segment (start 197.358 90.17) (end 191.262 90.17) (width 0.25) (layer "B.Cu") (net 22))
 (segment (start 191.32 91.128) (end 197.358 85.09) (width 0.25) (layer "F.Cu") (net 20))
 (segment (start 181.158 88.76) (end 181.158 90.351604) (width 0.25) (layer "F.Cu") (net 20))
 (segment (start 198.628 86.36) (end 197.358 85.09) (width 0.25) (layer "F.Cu") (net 20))
 (segment (start 207.772 86.36) (end 198.628 86.36) (width 0.25) (layer "F.Cu") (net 20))
 (segment (start 181.158 90.351604) (end 181.934396 91.128) (width 0.25) (layer "F.Cu") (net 20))
 (segment (start 181.934396 91.128) (end 191.32 91.128) (width 0.25) (layer "F.Cu") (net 20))
 (segment (start 182.120792 90.678) (end 191.008 90.678) (width 0.25) (layer "F.Cu") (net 21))
 (segment (start 181.608 90.165208) (end 182.120792 90.678) (width 0.25) (layer "F.Cu") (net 21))
 (segment (start 201.168 83.82) (end 197.358 80.01) (width 0.25) (layer "F.Cu") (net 21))
 (segment (start 181.608 88.76) (end 181.608 90.165208) (width 0.25) (layer "F.Cu") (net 21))
 (segment (start 194.818 82.55) (end 197.358 80.01) (width 0.25) (layer "F.Cu") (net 21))
 (segment (start 194.818 86.868) (end 194.818 82.55) (width 0.25) (layer "F.Cu") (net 21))
 (segment (start 191.008 90.678) (end 194.818 86.868) (width 0.25) (layer "F.Cu") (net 21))
 (segment (start 207.772 83.82) (end 201.168 83.82) (width 0.25) (layer "F.Cu") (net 21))
 (segment (start 199.136 72.39) (end 199.898 73.152) (width 0.25) (layer "F.Cu") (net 31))
 (segment (start 179.358 84.86) (end 179.358 83.82) (width 0.25) (layer "F.Cu") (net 31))
 (segment (start 203.2 81.28) (end 207.772 81.28) (width 0.25) (layer "F.Cu") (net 31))
 (segment (start 199.898 73.152) (end 199.898 77.978) (width 0.25) (layer "F.Cu") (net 31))
 (segment (start 179.358 83.82) (end 179.358 77.944) (width 0.25) (layer "F.Cu") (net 31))
 (segment (start 179.358 77.944) (end 184.912 72.39) (width 0.25) (layer "F.Cu") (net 31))
 (segment (start 199.898 77.978) (end 203.2 81.28) (width 0.25) (layer "F.Cu") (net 31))
 (segment (start 184.912 72.39) (end 199.136 72.39) (width 0.25) (layer "F.Cu") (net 31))
 (segment (start 180.258 90.85) (end 180.258 88.76) (width 0.25) (layer "F.Cu") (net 18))
 (segment (start 209.55 92.964) (end 209.296 93.218) (width 0.25) (layer "F.Cu") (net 18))
 (segment (start 209.55 77.978) (end 209.55 92.964) (width 0.25) (layer "F.Cu") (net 18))
 (segment (start 182.626 93.218) (end 180.258 90.85) (width 0.25) (layer "F.Cu") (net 18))
 (segment (start 207.772 76.2) (end 209.55 77.978) (width 0.25) (layer "F.Cu") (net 18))
 (segment (start 209.296 93.218) (end 182.626 93.218) (width 0.25) (layer "F.Cu") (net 18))
 (segment (start 212.3785 73.66) (end 207.772 73.66) (width 0.25) (layer "F.Cu") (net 15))
 (segment (start 215.7025 70.336) (end 212.3785 73.66) (width 0.25) (layer "F.Cu") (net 15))
 (segment (start 175.26 80.772) (end 178.908 84.42) (width 0.25) (layer "F.Cu") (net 17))
 (segment (start 172.72 80.772) (end 175.26 80.772) (width 0.25) (layer "F.Cu") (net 17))
 (segment (start 178.908 84.42) (end 178.908 84.86) (width 0.25) (layer "F.Cu") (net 17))
 (segment (start 179.358 96.554) (end 179.358 88.76) (width 0.25) (layer "F.Cu") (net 6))
 (segment (start 184.15 101.346) (end 179.358 96.554) (width 0.25) (layer "F.Cu") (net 6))
 (segment (start 184.15 106.68) (end 184.15 101.346) (width 0.25) (layer "F.Cu") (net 6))
 (segment (start 178.908 106.518) (end 178.908 88.76) (width 0.25) (layer "F.Cu") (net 7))
 (segment (start 179.07 106.68) (end 178.908 106.518) (width 0.25) (layer "F.Cu") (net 7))
 (segment (start 176.276 108.966) (end 186.69 108.966) (width 0.25) (layer "F.Cu") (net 8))
 (segment (start 179.808 93.754) (end 179.808 88.76) (width 0.25) (layer "F.Cu") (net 8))
 (segment (start 186.69 100.636) (end 179.808 93.754) (width 0.25) (layer "F.Cu") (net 8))
 (segment (start 173.99 106.68) (end 176.276 108.966) (width 0.25) (layer "F.Cu") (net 8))
 (segment (start 186.69 108.966) (end 186.69 100.636) (width 0.25) (layer "F.Cu") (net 8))
 (segment (start 178.308 85.91) (end 167.952 85.91) (width 0.25) (layer "F.Cu") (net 5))
 (segment (start 164.9965 84.582) (end 166.624 84.582) (width 0.25) (layer "F.Cu") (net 5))
 (segment (start 157.226 75.692) (end 165.1 83.566) (width 0.25) (layer "F.Cu") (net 5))
 (segment (start 165.1 83.566) (end 164.9965 83.6695) (width 0.25) (layer "F.Cu") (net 5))
 (segment (start 154.432 75.692) (end 157.226 75.692) (width 0.25) (layer "F.Cu") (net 5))
 (segment (start 164.9965 83.6695) (end 164.9965 84.582) (width 0.25) (layer "F.Cu") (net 5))
 (segment (start 166.624 84.582) (end 167.952 85.91) (width 0.25) (layer "F.Cu") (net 5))
 (segment (start 175.26 88.16) (end 175.006 88.414) (width 0.25) (layer "F.Cu") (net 9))
 (segment (start 178.308 88.16) (end 175.26 88.16) (width 0.25) (layer "F.Cu") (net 9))
 (segment (start 175.006 88.414) (end 175.006 93.218) (width 0.25) (layer "F.Cu") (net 9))
 (segment (start 180.258 81.362) (end 186.69 74.93) (width 0.25) (layer "F.Cu") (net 29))
 (segment (start 180.34 82.929604) (end 182.243604 81.026) (width 0.25) (layer "F.Cu") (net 29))
 (segment (start 182.243604 81.026) (end 182.9835 81.026) (width 0.25) (layer "F.Cu") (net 29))
 (segment (start 180.258 84.86) (end 180.258 81.362) (width 0.25) (layer "F.Cu") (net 29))
 (segment (start 186.69 74.93) (end 197.358 74.93) (width 0.25) (layer "F.Cu") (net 29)))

